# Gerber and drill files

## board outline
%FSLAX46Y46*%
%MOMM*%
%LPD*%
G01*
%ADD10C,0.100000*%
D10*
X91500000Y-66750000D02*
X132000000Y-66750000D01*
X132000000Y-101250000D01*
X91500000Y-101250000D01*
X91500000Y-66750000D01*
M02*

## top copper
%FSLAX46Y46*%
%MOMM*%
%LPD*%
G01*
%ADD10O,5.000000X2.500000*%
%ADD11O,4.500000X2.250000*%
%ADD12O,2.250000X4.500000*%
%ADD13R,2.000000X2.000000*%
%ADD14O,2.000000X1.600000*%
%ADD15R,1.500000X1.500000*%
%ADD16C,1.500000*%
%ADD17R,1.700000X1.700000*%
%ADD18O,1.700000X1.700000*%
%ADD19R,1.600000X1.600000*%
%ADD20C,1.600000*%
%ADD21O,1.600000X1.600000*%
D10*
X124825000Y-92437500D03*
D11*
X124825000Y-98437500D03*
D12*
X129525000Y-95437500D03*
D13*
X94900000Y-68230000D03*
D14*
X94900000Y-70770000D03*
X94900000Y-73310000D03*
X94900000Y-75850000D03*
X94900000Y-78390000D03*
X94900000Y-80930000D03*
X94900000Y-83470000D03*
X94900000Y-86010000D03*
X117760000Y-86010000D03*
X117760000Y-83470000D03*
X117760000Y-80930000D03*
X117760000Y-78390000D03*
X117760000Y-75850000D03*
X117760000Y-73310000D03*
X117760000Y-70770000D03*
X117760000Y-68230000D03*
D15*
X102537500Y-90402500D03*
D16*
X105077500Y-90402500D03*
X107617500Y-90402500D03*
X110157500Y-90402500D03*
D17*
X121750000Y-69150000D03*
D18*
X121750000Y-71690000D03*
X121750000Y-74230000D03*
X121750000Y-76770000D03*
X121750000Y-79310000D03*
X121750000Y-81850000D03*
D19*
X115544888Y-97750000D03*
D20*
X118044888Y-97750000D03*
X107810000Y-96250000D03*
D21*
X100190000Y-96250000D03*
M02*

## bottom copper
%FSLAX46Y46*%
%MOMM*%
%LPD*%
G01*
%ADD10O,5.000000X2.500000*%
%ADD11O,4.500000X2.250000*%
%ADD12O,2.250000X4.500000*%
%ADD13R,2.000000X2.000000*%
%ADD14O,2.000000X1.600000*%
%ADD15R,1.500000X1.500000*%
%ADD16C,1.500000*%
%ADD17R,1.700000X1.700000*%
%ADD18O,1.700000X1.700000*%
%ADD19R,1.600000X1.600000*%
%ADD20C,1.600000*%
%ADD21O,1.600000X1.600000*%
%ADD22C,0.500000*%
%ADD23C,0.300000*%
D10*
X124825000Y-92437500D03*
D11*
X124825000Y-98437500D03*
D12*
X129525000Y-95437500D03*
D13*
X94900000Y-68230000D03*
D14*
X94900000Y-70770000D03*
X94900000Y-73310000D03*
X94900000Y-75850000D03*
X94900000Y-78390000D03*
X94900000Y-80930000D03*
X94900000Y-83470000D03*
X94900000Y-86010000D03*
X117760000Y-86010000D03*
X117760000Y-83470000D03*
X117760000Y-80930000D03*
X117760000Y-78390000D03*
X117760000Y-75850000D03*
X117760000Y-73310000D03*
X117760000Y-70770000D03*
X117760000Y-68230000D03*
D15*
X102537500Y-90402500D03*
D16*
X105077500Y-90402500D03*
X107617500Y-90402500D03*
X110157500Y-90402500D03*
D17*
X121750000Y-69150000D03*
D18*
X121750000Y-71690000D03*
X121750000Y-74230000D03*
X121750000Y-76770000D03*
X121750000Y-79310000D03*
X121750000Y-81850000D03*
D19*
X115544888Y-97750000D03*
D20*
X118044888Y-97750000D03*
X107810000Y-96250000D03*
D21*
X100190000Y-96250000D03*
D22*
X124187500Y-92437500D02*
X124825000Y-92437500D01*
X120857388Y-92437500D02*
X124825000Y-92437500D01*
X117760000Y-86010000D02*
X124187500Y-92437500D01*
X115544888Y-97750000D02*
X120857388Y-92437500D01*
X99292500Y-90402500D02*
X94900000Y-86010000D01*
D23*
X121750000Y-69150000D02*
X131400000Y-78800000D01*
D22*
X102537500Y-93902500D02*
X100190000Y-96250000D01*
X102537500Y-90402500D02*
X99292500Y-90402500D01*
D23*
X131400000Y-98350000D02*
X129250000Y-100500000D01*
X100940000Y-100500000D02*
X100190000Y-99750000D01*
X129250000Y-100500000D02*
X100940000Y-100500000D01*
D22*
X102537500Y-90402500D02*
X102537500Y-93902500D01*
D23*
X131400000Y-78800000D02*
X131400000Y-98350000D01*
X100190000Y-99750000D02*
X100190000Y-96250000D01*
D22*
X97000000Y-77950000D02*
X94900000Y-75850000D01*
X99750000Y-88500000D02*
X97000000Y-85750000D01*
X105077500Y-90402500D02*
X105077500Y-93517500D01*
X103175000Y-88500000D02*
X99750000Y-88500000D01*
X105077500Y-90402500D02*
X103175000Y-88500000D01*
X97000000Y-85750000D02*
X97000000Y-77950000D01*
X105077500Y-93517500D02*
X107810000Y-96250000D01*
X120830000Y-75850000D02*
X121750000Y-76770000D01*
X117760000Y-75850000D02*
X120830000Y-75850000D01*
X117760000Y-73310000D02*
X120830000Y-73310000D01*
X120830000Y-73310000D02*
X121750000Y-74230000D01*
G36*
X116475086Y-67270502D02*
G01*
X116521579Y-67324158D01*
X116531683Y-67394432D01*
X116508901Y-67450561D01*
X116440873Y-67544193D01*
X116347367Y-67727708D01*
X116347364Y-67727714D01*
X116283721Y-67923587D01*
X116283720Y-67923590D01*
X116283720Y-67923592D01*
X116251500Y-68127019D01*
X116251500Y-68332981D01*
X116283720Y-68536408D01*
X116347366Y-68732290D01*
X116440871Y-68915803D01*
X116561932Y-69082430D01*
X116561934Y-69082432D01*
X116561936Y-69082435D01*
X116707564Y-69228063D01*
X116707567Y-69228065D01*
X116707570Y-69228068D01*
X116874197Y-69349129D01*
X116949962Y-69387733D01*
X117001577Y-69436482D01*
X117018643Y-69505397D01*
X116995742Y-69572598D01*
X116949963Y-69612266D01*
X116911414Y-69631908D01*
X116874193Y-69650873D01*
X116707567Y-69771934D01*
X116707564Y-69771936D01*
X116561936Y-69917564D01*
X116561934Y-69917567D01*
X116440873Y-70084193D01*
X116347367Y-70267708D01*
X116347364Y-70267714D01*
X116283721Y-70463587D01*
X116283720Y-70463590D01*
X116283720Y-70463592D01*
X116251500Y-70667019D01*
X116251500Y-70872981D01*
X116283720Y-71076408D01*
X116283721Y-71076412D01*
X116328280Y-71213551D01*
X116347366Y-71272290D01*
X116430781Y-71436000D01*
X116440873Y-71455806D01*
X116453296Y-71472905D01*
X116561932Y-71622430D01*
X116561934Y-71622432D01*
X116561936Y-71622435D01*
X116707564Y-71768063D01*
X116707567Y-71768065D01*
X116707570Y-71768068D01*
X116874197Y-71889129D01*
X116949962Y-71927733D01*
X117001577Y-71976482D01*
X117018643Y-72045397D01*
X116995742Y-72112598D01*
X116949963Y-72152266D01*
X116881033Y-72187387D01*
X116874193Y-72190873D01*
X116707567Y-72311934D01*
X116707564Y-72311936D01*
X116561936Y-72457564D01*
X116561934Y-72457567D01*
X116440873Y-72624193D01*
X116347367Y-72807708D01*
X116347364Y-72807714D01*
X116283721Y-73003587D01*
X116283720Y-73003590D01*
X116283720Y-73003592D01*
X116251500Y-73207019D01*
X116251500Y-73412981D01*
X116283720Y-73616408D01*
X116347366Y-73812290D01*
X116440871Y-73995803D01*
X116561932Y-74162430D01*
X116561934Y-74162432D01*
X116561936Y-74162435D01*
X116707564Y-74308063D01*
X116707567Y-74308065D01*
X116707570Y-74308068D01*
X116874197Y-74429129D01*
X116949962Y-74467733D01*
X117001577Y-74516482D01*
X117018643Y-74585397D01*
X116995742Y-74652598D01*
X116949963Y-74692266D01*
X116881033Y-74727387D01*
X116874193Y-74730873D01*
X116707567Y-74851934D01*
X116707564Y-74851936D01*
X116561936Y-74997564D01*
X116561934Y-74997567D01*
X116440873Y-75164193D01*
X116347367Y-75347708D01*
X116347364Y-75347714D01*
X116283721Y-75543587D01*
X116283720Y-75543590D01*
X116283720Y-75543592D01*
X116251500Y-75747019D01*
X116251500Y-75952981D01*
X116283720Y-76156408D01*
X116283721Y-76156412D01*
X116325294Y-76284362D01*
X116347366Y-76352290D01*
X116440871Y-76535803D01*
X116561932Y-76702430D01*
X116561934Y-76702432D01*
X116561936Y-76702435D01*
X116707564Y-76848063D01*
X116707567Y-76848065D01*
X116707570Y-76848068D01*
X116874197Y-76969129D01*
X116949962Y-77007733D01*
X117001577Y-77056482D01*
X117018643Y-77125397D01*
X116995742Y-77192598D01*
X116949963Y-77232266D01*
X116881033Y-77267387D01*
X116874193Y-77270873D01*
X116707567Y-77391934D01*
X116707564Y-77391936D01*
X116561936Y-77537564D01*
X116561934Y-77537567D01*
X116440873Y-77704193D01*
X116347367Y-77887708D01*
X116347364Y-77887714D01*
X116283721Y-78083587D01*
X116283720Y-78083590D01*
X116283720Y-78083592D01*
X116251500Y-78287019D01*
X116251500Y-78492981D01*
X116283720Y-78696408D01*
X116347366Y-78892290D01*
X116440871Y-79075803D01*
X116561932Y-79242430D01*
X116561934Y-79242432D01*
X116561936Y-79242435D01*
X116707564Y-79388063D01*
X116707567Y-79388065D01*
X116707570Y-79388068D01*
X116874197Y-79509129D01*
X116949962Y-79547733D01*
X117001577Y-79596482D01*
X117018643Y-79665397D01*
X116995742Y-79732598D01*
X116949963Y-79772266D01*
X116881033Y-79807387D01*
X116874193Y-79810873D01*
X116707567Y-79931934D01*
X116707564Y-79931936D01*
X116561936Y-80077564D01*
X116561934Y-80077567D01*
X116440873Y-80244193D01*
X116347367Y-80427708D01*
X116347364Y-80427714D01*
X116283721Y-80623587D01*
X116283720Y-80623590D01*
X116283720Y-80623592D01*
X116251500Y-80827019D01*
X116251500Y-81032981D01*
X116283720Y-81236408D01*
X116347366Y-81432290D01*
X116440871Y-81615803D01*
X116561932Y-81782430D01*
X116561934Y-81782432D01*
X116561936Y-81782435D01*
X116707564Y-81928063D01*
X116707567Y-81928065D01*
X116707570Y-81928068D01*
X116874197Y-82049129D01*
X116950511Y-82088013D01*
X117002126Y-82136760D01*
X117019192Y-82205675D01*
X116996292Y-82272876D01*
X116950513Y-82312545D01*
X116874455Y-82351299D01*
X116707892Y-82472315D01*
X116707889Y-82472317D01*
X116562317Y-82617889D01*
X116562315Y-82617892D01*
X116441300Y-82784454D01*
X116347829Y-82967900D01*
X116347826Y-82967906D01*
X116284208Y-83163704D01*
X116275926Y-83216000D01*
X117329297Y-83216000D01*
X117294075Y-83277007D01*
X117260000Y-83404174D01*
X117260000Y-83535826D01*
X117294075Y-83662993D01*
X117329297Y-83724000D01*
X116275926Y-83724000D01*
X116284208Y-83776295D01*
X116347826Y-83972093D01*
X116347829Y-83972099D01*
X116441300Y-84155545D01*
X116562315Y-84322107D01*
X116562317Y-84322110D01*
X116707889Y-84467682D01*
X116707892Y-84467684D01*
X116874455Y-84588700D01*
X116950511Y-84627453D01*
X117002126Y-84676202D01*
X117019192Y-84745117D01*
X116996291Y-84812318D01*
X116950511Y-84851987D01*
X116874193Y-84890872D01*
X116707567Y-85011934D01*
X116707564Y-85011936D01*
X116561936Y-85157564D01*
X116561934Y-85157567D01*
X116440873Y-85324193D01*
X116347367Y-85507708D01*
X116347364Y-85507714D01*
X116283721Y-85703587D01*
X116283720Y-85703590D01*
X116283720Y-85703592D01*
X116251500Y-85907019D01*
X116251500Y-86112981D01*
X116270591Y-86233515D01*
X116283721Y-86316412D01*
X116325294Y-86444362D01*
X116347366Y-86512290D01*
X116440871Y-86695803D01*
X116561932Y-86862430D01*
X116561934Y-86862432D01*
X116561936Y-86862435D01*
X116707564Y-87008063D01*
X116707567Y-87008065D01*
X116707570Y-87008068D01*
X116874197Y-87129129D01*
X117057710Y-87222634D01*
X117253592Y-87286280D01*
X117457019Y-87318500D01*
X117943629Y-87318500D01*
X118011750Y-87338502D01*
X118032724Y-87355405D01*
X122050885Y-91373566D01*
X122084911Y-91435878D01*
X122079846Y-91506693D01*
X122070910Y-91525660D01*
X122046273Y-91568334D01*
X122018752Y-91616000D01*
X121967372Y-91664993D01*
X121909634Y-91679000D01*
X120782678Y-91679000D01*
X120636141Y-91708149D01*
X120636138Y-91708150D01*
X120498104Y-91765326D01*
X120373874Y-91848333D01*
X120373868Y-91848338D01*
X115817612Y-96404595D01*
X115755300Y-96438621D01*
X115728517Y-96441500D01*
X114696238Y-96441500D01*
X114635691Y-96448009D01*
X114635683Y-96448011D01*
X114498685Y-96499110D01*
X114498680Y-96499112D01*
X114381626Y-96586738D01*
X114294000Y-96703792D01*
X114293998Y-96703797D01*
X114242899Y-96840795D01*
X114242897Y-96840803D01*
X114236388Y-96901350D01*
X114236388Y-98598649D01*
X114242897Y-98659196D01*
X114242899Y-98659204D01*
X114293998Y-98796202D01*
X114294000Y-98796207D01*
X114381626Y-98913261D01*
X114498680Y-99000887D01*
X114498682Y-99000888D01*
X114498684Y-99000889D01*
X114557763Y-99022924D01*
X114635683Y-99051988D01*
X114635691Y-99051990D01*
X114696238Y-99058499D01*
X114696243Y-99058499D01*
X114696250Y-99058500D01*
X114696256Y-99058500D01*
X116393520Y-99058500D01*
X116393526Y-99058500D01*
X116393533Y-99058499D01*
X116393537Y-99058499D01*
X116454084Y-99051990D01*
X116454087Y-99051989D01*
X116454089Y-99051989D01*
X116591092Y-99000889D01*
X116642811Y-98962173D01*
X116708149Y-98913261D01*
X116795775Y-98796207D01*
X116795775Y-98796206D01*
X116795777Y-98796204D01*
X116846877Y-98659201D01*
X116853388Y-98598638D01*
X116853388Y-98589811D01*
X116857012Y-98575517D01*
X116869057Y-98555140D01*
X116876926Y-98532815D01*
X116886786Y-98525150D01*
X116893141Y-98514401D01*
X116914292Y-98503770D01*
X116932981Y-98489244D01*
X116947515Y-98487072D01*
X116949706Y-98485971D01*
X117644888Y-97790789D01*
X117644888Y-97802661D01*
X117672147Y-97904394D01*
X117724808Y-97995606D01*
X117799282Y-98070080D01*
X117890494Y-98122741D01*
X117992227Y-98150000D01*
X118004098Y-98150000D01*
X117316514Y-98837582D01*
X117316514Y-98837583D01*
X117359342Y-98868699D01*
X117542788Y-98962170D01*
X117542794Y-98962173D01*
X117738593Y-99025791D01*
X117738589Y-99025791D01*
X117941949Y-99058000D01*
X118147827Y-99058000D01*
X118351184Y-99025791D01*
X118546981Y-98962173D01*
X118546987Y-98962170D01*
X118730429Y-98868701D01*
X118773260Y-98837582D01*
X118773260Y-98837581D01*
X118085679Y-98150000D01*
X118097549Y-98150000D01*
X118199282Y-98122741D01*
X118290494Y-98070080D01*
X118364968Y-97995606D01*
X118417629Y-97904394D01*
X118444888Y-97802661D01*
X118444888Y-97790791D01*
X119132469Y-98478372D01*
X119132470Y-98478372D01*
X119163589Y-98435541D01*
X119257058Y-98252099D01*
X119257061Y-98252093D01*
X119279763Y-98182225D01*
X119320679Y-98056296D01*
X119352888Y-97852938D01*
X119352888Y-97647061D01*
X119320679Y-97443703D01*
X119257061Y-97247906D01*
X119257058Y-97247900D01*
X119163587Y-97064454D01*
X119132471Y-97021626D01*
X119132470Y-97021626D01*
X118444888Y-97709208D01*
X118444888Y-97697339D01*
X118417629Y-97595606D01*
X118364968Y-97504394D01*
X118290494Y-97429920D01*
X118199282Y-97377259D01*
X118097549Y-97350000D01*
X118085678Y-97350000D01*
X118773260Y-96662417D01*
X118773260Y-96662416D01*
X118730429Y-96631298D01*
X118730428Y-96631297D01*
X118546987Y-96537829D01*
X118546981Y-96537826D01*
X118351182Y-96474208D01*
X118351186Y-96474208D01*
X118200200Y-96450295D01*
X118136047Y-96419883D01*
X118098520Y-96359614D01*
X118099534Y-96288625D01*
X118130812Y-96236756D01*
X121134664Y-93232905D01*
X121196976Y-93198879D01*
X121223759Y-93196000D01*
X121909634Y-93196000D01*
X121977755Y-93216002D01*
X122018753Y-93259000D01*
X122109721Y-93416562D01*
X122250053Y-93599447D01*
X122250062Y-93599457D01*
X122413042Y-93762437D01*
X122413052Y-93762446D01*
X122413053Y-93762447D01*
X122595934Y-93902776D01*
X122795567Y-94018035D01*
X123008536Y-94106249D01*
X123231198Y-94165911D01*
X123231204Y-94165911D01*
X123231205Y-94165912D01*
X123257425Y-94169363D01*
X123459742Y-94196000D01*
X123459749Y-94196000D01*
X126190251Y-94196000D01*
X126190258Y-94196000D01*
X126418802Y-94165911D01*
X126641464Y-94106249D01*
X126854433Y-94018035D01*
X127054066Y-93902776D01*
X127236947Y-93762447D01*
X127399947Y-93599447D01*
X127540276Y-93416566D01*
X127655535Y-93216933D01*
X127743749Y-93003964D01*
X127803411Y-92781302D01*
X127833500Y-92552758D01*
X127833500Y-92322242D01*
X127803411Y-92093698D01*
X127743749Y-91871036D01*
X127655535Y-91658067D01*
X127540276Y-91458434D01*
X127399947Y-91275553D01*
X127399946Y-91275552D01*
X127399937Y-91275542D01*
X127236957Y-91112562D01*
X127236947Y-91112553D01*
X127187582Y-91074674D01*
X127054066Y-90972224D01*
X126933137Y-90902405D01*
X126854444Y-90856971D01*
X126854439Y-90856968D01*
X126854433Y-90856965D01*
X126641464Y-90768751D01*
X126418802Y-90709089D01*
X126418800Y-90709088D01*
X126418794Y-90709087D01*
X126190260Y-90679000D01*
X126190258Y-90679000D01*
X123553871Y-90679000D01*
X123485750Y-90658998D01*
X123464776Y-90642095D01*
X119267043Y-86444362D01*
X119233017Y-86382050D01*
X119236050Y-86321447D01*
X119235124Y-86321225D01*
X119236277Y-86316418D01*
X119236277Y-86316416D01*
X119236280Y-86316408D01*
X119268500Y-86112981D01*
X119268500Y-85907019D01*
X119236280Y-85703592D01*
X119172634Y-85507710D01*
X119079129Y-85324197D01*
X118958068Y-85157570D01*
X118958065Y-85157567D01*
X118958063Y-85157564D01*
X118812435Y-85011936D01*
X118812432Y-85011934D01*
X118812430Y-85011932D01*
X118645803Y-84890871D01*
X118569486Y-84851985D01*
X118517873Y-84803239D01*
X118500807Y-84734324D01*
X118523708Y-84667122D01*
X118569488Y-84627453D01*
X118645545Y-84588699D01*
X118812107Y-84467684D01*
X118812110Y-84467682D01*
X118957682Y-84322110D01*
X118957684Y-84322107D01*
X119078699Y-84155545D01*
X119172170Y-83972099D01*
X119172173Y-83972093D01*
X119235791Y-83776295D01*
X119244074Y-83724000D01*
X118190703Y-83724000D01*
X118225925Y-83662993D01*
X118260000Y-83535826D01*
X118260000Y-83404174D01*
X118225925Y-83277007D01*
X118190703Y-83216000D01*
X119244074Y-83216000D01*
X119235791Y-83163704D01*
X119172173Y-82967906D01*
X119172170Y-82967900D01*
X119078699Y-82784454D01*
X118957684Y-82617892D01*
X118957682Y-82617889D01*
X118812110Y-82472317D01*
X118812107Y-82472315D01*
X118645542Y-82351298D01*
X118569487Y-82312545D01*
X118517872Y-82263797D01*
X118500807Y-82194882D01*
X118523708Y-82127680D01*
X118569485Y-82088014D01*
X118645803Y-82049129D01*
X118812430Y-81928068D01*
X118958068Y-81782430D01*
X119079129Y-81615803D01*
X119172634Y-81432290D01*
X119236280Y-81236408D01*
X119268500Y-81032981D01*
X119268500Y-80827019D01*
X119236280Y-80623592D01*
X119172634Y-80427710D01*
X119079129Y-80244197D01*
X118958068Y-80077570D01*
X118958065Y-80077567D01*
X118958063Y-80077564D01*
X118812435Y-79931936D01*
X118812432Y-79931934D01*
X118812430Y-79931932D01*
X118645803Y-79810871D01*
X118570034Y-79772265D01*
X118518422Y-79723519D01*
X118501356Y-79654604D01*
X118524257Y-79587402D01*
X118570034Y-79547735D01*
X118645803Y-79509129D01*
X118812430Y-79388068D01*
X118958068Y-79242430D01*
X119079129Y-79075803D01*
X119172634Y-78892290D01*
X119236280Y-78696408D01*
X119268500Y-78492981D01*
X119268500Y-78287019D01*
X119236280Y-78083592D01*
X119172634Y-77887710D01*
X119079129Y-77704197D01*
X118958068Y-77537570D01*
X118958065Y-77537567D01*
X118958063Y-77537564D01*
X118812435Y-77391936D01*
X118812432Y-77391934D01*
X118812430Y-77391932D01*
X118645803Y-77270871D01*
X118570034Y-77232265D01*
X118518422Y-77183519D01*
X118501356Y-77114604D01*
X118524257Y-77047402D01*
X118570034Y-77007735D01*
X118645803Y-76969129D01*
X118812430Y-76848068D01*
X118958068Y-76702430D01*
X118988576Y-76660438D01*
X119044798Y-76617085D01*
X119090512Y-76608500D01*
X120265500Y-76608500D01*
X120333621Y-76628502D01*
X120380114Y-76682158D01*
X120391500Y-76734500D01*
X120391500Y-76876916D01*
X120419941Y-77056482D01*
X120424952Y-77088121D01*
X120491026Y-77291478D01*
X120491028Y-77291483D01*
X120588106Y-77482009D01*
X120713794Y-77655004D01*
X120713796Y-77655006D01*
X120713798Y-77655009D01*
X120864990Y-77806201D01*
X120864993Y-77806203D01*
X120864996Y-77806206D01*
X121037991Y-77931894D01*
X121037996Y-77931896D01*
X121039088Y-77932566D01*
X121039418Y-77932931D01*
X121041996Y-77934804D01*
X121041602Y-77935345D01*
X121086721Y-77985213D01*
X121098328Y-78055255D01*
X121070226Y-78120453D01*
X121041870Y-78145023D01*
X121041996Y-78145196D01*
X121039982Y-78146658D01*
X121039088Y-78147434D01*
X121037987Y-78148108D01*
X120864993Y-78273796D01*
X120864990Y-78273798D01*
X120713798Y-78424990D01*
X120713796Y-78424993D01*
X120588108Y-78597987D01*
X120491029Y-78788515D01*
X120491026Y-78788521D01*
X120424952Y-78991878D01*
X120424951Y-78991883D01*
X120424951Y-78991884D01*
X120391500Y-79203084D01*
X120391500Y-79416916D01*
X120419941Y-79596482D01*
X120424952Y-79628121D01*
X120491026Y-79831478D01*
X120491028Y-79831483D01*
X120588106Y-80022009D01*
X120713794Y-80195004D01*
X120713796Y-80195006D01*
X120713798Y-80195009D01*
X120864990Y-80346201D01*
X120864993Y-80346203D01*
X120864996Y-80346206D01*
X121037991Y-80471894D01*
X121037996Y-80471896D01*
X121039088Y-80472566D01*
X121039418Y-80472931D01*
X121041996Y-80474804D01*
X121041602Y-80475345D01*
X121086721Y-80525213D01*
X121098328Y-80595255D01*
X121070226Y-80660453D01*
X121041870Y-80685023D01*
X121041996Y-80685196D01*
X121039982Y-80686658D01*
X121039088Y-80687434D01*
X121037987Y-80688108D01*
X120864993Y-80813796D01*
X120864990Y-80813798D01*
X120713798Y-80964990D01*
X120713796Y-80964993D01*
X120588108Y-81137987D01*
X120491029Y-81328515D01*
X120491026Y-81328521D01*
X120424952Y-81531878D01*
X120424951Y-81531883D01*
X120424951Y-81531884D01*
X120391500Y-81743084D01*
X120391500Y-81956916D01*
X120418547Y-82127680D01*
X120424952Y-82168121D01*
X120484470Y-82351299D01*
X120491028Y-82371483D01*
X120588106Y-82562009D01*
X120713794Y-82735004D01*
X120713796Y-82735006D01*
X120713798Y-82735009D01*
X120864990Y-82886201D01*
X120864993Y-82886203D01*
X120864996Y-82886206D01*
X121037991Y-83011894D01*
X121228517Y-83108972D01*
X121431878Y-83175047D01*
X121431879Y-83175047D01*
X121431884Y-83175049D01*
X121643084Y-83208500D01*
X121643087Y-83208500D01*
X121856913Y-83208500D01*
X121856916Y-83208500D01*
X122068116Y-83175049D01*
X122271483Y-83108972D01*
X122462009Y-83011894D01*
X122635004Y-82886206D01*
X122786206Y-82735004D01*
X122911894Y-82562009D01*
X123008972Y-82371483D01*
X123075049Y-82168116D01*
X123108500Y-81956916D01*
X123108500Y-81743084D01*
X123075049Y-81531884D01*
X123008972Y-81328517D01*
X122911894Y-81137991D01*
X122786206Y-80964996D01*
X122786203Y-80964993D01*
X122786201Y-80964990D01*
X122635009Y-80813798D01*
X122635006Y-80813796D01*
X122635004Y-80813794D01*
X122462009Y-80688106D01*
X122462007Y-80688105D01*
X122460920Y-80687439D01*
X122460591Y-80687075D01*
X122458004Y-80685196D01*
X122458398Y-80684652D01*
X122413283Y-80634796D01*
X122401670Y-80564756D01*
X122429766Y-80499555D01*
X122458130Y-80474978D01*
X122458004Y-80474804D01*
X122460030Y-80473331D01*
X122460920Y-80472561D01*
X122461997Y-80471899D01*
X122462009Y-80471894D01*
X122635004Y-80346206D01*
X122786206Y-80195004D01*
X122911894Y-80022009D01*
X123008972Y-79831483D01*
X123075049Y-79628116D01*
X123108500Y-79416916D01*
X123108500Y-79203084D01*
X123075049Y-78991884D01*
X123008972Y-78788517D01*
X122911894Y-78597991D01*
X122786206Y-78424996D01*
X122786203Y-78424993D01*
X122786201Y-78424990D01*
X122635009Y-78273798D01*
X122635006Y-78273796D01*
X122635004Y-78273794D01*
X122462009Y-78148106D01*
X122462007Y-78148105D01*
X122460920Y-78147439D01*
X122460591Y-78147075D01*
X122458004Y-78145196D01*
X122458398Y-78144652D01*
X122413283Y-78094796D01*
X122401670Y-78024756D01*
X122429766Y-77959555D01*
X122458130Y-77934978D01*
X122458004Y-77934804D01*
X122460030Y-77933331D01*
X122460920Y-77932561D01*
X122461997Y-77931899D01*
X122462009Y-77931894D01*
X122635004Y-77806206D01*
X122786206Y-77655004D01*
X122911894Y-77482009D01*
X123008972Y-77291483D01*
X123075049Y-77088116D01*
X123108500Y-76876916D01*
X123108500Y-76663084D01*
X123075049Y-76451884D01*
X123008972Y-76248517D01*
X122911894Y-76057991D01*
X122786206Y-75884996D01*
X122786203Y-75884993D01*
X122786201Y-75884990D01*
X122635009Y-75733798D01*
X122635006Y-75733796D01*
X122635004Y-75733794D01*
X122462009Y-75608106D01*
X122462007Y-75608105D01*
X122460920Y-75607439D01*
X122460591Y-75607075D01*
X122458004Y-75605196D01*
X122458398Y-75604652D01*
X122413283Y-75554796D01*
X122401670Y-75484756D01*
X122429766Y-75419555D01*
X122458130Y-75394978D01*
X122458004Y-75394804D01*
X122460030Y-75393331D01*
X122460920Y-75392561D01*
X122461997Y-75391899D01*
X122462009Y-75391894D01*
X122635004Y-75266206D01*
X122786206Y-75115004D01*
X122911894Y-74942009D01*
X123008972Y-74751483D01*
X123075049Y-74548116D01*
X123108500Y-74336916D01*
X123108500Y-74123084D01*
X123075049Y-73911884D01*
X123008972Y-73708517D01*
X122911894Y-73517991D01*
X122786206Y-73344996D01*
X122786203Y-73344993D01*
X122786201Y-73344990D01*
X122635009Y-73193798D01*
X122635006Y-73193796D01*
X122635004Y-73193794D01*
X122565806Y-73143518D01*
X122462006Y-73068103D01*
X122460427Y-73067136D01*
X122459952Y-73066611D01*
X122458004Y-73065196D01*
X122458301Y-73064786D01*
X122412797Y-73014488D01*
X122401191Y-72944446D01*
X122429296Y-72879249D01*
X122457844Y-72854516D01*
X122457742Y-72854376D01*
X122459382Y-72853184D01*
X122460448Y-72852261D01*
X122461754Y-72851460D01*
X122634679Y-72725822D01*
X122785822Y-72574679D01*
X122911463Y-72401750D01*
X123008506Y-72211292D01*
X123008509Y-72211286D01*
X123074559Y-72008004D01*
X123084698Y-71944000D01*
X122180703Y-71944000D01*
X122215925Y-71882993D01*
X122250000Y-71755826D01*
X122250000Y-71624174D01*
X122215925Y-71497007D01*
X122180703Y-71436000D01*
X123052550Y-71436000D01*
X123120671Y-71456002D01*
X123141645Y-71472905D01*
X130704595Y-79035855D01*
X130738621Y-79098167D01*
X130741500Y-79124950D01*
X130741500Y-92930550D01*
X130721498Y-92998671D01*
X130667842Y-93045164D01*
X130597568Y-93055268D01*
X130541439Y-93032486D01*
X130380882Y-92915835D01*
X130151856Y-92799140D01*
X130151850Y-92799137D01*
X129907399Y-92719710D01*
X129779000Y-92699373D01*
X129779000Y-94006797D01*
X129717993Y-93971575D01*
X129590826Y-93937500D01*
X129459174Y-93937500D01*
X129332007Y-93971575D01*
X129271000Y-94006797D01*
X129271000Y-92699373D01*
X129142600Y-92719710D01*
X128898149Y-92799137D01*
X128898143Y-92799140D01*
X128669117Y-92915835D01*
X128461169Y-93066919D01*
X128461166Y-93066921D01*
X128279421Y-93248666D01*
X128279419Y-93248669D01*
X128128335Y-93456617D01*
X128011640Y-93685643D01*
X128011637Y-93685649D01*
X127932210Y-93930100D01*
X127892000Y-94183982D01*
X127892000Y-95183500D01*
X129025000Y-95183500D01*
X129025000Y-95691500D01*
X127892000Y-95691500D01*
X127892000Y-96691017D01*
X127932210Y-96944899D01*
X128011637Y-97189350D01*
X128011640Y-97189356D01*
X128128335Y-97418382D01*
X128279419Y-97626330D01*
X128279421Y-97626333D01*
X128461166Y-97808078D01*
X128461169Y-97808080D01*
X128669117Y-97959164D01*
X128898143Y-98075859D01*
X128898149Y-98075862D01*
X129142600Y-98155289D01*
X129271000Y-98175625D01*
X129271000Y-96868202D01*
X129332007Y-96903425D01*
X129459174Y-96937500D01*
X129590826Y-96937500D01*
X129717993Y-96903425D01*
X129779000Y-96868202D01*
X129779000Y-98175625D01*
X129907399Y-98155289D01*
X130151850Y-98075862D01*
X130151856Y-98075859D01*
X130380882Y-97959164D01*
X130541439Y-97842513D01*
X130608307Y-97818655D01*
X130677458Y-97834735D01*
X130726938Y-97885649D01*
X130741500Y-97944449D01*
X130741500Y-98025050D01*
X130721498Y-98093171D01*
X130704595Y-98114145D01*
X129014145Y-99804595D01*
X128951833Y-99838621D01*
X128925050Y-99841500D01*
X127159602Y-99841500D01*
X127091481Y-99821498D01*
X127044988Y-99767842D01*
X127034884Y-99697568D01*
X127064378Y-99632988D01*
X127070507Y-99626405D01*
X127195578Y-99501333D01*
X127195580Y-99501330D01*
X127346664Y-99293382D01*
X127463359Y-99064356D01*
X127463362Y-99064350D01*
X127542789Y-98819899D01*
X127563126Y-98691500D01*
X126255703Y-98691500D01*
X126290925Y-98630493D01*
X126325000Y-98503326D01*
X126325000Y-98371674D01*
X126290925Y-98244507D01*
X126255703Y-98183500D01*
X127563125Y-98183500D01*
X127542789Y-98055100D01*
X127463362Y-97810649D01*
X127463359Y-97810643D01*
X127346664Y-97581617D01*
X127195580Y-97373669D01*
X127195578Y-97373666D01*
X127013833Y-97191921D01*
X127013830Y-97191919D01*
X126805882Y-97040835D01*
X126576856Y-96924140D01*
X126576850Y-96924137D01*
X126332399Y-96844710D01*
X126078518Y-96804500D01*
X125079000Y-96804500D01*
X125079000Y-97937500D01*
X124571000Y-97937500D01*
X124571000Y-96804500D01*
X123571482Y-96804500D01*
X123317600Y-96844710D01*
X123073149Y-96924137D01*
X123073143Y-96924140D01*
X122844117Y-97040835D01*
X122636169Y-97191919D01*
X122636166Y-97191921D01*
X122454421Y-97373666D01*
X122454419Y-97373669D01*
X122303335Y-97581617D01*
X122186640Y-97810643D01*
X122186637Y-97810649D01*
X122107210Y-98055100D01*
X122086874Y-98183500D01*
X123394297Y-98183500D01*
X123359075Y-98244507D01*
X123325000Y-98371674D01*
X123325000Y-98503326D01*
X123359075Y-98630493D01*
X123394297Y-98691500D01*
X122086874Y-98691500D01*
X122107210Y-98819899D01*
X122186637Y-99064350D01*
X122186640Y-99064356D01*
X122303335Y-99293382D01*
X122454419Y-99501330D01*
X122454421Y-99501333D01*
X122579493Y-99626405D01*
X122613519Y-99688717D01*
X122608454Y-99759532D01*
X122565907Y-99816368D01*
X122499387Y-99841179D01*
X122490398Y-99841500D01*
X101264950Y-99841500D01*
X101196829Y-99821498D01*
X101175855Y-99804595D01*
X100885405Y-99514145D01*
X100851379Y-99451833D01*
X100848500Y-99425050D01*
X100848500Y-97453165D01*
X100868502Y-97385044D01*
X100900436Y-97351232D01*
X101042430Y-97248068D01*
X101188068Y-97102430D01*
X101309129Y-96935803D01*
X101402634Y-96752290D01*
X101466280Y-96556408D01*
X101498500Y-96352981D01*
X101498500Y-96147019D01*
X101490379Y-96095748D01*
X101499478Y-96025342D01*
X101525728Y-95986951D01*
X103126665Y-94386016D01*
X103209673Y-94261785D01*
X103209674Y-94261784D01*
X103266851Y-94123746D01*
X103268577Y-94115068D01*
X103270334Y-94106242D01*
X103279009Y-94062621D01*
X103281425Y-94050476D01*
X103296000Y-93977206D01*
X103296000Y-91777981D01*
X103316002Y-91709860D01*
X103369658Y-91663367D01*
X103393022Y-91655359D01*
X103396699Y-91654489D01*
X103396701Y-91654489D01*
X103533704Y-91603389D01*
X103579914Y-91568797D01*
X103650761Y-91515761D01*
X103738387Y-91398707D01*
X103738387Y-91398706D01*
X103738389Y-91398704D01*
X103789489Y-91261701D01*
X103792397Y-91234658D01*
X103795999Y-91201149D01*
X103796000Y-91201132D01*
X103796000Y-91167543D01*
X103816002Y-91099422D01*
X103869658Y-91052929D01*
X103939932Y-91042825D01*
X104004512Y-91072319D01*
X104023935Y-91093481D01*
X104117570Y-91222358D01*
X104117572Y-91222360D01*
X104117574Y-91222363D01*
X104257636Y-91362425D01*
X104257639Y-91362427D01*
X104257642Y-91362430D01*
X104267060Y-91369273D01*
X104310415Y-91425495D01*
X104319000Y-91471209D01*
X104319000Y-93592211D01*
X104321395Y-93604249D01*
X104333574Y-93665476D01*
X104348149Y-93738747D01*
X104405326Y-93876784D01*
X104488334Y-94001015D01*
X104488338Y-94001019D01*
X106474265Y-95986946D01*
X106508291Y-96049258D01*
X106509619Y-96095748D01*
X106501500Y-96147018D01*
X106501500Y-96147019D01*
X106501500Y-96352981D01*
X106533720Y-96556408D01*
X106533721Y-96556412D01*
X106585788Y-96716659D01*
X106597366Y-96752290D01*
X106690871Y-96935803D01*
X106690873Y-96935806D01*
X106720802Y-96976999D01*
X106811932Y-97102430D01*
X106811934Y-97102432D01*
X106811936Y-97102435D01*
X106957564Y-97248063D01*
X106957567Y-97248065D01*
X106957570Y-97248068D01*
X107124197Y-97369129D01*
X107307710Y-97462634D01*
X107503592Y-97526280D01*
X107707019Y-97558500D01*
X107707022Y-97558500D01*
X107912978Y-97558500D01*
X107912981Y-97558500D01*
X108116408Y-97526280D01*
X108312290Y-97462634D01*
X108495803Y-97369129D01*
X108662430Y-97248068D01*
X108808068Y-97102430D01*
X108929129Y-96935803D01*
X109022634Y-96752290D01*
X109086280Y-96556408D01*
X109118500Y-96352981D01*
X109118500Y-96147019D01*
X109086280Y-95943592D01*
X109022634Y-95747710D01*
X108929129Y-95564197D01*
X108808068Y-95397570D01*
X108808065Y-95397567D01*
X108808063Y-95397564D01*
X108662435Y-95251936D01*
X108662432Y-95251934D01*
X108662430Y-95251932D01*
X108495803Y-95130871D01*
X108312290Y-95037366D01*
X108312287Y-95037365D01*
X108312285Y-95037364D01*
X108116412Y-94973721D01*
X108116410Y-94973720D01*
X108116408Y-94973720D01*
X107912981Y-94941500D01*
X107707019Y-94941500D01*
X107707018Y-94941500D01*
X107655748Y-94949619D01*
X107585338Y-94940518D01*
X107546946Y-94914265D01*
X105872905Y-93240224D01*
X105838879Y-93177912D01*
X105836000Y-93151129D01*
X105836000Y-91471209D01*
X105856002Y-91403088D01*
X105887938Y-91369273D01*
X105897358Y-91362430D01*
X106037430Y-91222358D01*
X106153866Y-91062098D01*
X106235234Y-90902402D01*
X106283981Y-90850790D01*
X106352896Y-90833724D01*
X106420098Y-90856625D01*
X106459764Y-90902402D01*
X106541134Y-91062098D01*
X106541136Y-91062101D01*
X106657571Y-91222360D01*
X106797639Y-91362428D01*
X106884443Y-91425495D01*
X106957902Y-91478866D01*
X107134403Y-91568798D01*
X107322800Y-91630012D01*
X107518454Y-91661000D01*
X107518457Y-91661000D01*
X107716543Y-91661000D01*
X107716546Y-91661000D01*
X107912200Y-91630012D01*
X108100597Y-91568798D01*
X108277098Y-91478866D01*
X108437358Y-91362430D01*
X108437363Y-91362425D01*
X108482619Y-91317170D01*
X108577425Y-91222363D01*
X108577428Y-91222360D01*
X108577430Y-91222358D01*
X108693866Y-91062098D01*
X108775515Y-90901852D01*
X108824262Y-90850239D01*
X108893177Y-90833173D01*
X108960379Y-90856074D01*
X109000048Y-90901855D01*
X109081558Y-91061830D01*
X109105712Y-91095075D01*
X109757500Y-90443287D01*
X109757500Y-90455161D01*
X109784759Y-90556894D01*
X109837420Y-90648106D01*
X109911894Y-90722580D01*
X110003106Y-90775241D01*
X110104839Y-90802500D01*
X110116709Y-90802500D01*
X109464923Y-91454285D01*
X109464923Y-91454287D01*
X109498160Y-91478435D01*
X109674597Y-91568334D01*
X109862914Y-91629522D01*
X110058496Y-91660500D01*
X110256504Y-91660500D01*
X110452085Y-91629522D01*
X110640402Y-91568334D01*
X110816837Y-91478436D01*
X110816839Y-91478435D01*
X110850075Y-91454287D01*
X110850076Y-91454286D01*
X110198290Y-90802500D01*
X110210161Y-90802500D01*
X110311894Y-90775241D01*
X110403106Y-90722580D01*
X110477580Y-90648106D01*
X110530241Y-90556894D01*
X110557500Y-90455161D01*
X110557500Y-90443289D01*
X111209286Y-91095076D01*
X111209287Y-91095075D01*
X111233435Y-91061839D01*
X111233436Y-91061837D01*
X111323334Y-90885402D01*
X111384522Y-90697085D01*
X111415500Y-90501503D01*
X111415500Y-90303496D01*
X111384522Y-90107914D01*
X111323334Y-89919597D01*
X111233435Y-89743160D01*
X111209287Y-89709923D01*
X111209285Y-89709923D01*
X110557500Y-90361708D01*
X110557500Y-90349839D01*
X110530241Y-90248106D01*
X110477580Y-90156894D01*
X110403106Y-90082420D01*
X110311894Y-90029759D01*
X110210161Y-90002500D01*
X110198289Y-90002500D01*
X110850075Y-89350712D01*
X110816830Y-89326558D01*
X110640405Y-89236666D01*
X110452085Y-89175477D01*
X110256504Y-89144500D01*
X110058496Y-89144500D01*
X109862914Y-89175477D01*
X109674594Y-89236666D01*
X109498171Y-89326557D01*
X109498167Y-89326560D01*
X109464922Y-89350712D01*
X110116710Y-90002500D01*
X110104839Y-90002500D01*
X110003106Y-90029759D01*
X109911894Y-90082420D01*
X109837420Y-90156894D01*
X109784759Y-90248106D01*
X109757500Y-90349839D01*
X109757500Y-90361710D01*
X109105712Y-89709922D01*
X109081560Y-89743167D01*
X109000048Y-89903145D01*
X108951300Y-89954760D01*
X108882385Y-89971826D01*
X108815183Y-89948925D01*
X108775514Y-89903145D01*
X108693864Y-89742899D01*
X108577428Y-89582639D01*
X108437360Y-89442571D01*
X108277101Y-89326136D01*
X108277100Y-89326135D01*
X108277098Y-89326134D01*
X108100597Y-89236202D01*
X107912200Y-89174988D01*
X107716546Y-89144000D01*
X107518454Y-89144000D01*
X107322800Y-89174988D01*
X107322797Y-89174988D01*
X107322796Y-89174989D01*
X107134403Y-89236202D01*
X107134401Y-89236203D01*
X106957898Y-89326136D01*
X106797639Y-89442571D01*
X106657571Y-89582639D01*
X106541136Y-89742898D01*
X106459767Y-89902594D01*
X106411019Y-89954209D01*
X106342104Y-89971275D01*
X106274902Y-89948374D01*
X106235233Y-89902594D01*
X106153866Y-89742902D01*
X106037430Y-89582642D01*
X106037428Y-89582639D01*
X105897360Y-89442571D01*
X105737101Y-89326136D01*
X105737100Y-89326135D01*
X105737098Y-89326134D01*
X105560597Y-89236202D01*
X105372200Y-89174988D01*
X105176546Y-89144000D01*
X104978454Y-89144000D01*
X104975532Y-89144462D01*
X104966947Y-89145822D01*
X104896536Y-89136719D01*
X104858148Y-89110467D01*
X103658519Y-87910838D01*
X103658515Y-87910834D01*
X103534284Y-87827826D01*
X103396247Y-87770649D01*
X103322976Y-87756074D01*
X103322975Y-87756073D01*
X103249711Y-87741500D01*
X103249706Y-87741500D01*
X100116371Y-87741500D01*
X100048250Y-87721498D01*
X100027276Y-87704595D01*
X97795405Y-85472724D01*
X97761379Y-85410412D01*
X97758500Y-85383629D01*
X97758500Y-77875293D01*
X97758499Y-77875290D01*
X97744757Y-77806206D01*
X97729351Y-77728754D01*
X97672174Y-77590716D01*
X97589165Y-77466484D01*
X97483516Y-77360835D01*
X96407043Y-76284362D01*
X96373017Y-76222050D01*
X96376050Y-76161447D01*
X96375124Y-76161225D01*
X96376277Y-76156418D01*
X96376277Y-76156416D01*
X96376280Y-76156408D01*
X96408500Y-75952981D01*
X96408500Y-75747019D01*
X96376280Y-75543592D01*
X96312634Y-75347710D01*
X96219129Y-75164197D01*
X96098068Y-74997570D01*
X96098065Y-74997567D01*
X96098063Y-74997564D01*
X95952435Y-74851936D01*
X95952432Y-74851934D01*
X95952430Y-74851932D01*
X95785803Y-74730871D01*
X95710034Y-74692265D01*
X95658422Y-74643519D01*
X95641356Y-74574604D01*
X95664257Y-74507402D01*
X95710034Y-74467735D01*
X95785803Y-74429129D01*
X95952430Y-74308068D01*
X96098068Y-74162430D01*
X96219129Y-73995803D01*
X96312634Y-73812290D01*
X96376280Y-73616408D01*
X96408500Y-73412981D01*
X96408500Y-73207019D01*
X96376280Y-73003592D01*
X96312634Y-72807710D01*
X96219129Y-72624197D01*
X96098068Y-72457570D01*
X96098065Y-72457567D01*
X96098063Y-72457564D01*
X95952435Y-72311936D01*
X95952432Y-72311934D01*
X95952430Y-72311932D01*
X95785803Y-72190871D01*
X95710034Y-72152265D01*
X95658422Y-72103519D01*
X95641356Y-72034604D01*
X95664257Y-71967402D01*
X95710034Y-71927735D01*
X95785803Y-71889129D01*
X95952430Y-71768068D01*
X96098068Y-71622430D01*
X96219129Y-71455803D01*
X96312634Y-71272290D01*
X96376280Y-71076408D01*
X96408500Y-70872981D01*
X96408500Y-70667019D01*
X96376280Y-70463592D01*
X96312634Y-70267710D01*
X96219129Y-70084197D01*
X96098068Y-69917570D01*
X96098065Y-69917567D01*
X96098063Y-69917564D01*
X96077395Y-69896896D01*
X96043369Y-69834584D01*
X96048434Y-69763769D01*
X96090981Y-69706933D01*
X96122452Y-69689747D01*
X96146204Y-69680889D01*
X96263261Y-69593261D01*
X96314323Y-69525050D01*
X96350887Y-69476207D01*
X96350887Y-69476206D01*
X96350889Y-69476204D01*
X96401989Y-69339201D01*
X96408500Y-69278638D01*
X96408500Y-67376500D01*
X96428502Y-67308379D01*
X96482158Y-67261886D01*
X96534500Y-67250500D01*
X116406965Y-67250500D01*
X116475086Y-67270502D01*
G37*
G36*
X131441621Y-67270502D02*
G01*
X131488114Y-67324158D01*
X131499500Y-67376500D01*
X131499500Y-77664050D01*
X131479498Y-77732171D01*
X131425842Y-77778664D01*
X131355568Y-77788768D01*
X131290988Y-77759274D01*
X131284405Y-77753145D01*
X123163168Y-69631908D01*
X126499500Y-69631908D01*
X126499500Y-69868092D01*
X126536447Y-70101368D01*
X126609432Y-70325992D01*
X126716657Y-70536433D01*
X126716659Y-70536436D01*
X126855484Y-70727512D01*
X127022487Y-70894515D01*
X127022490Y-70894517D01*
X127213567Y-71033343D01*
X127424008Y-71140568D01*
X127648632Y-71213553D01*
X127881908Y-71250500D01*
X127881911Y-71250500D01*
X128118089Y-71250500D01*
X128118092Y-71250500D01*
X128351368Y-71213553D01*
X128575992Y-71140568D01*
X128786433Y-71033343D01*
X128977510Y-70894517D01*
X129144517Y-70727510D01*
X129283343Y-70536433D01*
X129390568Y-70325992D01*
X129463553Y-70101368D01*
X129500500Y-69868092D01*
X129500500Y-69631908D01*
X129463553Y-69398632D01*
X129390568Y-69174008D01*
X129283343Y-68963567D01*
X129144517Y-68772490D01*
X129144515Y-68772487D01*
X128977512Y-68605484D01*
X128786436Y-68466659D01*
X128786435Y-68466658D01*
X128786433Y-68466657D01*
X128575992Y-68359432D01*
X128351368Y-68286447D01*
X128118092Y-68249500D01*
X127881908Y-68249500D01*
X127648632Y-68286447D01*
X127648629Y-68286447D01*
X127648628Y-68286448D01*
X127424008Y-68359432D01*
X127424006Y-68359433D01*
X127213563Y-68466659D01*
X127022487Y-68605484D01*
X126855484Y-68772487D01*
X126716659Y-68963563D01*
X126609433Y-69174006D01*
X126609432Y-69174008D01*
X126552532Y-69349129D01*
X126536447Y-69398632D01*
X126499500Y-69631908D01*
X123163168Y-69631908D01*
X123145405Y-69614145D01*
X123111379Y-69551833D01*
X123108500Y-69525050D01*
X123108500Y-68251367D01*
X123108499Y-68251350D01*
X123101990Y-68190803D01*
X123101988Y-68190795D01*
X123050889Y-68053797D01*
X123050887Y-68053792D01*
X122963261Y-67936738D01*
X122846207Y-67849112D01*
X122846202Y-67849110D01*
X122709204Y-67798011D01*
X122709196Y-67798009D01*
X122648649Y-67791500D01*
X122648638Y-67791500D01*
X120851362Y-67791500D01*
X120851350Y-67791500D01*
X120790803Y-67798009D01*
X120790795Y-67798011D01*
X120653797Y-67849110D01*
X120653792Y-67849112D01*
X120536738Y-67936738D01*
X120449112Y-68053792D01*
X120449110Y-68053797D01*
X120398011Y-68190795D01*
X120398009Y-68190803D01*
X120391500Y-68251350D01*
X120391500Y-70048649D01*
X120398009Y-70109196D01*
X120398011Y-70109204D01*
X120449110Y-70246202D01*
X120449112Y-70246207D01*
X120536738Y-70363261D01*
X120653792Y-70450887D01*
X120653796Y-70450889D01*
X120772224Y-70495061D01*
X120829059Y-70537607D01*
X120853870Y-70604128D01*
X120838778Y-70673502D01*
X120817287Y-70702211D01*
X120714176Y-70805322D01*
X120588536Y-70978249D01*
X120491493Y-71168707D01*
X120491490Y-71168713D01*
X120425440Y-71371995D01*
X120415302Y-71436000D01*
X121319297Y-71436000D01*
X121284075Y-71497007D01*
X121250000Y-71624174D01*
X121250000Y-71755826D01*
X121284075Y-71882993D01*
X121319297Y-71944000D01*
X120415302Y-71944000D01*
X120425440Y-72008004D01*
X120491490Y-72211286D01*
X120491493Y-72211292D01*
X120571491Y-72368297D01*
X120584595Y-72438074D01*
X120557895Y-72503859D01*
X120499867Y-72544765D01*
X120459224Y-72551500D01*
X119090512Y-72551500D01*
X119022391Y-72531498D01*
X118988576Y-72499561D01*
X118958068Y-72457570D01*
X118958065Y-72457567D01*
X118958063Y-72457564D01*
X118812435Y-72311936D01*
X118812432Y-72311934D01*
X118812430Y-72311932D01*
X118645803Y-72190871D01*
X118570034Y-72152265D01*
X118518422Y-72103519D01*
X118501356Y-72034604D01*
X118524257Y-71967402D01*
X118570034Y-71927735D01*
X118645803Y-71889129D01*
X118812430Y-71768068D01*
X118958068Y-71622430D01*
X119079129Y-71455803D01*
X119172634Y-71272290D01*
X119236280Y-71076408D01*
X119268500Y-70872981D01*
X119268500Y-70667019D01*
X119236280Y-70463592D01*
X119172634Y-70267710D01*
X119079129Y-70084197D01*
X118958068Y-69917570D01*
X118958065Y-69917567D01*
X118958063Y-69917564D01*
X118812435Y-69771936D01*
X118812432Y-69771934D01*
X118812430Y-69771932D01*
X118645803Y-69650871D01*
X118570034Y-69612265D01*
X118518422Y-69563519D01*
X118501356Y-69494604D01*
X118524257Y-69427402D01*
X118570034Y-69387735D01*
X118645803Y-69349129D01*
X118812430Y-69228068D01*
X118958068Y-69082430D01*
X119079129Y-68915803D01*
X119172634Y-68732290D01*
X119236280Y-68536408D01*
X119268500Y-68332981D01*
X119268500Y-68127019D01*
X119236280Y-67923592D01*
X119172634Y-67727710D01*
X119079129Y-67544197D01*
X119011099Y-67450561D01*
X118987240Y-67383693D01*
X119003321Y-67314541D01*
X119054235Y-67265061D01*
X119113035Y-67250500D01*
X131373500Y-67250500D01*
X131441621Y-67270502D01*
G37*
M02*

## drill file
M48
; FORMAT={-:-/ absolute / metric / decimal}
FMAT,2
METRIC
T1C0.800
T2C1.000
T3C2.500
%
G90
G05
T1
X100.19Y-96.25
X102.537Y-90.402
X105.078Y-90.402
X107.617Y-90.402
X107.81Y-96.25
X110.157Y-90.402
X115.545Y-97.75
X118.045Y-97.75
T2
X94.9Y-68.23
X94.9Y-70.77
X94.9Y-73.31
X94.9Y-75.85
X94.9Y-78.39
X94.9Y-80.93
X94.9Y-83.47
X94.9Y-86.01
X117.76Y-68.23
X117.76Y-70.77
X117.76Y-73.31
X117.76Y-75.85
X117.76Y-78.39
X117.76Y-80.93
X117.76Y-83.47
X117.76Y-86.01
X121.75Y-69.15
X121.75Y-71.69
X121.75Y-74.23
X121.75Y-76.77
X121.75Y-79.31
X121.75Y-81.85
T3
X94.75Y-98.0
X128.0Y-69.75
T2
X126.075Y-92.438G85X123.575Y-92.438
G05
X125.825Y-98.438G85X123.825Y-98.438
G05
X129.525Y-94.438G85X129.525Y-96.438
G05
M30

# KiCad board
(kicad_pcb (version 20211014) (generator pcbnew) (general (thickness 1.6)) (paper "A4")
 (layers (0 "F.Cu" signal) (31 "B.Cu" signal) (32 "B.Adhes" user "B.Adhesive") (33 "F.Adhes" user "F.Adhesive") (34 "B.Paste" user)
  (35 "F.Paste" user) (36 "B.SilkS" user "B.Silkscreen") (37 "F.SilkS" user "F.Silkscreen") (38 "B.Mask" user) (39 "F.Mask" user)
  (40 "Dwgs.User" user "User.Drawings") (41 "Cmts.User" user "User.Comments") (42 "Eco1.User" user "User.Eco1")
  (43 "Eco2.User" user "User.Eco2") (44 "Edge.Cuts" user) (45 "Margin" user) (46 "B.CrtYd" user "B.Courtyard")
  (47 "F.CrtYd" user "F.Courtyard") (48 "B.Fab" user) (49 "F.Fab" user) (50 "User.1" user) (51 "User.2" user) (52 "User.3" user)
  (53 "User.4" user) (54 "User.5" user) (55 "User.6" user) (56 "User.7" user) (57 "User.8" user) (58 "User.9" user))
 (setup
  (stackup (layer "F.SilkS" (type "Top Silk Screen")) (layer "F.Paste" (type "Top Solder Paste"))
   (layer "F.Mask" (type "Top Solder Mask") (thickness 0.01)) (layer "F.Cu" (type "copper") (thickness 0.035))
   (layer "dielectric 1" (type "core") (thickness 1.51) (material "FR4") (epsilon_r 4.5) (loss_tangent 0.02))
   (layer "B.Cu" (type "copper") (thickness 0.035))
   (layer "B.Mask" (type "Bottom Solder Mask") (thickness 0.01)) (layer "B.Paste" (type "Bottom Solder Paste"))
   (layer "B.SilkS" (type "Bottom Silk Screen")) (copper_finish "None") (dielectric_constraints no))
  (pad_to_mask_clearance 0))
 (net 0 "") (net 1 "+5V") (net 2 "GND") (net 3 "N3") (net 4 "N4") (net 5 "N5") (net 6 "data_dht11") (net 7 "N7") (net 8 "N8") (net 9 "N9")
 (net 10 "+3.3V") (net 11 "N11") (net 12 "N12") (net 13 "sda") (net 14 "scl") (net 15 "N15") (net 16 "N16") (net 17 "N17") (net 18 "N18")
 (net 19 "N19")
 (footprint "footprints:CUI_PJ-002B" (layer "F.Cu") (at 124.825 92.4375 -90)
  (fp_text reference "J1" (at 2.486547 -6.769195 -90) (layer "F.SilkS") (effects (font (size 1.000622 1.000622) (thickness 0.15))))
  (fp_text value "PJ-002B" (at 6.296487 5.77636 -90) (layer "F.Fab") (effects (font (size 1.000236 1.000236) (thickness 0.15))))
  (pad "1" thru_hole oval locked (at 0 0 270) (size 2.5 5) (drill oval 1 3.5) (layers *.Cu *.Mask) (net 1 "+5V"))
  (pad "2" thru_hole oval locked (at 6 0 270) (size 2.25 4.5) (drill oval 1 3) (layers *.Cu *.Mask) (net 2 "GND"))
  (pad "3" thru_hole oval locked (at 3 -4.7 270) (size 4.5 2.25) (drill oval 3 1) (layers *.Cu *.Mask) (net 2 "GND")))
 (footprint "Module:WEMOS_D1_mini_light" (layer "F.Cu") (at 94.9 68.23)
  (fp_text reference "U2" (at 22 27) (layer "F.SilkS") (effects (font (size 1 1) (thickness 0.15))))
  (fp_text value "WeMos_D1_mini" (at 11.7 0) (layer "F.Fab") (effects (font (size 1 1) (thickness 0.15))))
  (pad "1" thru_hole rect (at 0 0) (size 2 2) (drill 1) (layers *.Cu *.Mask) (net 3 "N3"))
  (pad "2" thru_hole oval (at 0 2.54) (size 2 1.6) (drill 1) (layers *.Cu *.Mask) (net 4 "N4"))
  (pad "3" thru_hole oval (at 0 5.08) (size 2 1.6) (drill 1) (layers *.Cu *.Mask) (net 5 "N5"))
  (pad "4" thru_hole oval (at 0 7.62) (size 2 1.6) (drill 1) (layers *.Cu *.Mask) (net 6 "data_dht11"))
  (pad "5" thru_hole oval (at 0 10.16) (size 2 1.6) (drill 1) (layers *.Cu *.Mask) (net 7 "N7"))
  (pad "6" thru_hole oval (at 0 12.7) (size 2 1.6) (drill 1) (layers *.Cu *.Mask) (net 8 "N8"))
  (pad "7" thru_hole oval (at 0 15.24) (size 2 1.6) (drill 1) (layers *.Cu *.Mask) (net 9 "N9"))
  (pad "8" thru_hole oval (at 0 17.78) (size 2 1.6) (drill 1) (layers *.Cu *.Mask) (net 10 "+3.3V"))
  (pad "9" thru_hole oval (at 22.86 17.78) (size 2 1.6) (drill 1) (layers *.Cu *.Mask) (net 1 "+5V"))
  (pad "10" thru_hole oval (at 22.86 15.24) (size 2 1.6) (drill 1) (layers *.Cu *.Mask) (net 2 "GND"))
  (pad "11" thru_hole oval (at 22.86 12.7) (size 2 1.6) (drill 1) (layers *.Cu *.Mask) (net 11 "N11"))
  (pad "12" thru_hole oval (at 22.86 10.16) (size 2 1.6) (drill 1) (layers *.Cu *.Mask) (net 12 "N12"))
  (pad "13" thru_hole oval (at 22.86 7.62) (size 2 1.6) (drill 1) (layers *.Cu *.Mask) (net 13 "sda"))
  (pad "14" thru_hole oval (at 22.86 5.08) (size 2 1.6) (drill 1) (layers *.Cu *.Mask) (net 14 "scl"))
  (pad "15" thru_hole oval (at 22.86 2.54) (size 2 1.6) (drill 1) (layers *.Cu *.Mask) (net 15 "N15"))
  (pad "16" thru_hole oval (at 22.86 0) (size 2 1.6) (drill 1) (layers *.Cu *.Mask) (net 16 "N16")))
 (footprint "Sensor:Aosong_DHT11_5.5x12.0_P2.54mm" (layer "F.Cu") (at 102.5375 90.4025 90)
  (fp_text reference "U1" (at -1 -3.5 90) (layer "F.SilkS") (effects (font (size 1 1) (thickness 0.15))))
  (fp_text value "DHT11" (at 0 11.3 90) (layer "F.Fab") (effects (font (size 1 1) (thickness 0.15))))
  (pad "1" thru_hole rect (at 0 0 90) (size 1.5 1.5) (drill 0.8) (layers *.Cu *.Mask) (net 10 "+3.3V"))
  (pad "2" thru_hole circle (at 0 2.54 90) (size 1.5 1.5) (drill 0.8) (layers *.Cu *.Mask) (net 6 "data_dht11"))
  (pad "3" thru_hole circle (at 0 5.08 90) (size 1.5 1.5) (drill 0.8) (layers *.Cu *.Mask) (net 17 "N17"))
  (pad "4" thru_hole circle (at 0 7.62 90) (size 1.5 1.5) (drill 0.8) (layers *.Cu *.Mask) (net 2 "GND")))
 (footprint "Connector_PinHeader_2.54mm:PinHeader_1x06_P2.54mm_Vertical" (layer "F.Cu") (at 121.75 69.15)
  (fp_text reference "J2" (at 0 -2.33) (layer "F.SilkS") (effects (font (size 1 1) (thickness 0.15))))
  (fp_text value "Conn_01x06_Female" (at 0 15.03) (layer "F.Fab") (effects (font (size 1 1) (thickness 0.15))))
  (pad "1" thru_hole rect (at 0 0) (size 1.7 1.7) (drill 1) (layers *.Cu *.Mask) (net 10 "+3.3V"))
  (pad "2" thru_hole oval (at 0 2.54) (size 1.7 1.7) (drill 1) (layers *.Cu *.Mask) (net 2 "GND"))
  (pad "3" thru_hole oval (at 0 5.08) (size 1.7 1.7) (drill 1) (layers *.Cu *.Mask) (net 14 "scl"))
  (pad "4" thru_hole oval (at 0 7.62) (size 1.7 1.7) (drill 1) (layers *.Cu *.Mask) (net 13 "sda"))
  (pad "5" thru_hole oval (at 0 10.16) (size 1.7 1.7) (drill 1) (layers *.Cu *.Mask) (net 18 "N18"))
  (pad "6" thru_hole oval (at 0 12.7) (size 1.7 1.7) (drill 1) (layers *.Cu *.Mask) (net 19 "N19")))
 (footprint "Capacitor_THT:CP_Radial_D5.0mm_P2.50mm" (layer "F.Cu") (at 115.544888 97.75)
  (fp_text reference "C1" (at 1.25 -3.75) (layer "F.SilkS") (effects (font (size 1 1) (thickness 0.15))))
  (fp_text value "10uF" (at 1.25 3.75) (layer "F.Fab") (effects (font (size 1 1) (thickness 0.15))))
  (pad "1" thru_hole rect (at 0 0) (size 1.6 1.6) (drill 0.8) (layers *.Cu *.Mask) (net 1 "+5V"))
  (pad "2" thru_hole circle (at 2.5 0) (size 1.6 1.6) (drill 0.8) (layers *.Cu *.Mask) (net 2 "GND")))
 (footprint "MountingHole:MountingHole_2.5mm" (layer "F.Cu") (at 94.75 98)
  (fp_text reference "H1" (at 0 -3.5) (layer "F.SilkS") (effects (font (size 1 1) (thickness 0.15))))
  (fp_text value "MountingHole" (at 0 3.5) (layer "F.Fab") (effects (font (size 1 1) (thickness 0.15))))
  (pad "" np_thru_hole circle (at 0 0) (size 2.5 2.5) (drill 2.5) (layers *.Cu *.Mask)))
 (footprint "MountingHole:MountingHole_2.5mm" (layer "F.Cu") (at 128 69.75)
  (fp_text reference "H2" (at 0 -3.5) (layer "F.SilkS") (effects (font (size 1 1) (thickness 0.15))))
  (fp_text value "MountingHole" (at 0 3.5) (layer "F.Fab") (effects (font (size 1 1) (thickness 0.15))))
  (pad "" np_thru_hole circle (at 0 0) (size 2.5 2.5) (drill 2.5) (layers *.Cu *.Mask)))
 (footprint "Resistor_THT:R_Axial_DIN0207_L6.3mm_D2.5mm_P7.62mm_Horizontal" (layer "F.Cu") (at 107.81 96.25 180)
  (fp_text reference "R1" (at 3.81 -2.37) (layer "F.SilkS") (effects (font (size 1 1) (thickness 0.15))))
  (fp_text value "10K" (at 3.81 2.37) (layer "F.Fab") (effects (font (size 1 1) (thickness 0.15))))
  (pad "1" thru_hole circle (at 0 0 180) (size 1.6 1.6) (drill 0.8) (layers *.Cu *.Mask) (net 6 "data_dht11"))
  (pad "2" thru_hole oval (at 7.62 0 180) (size 1.6 1.6) (drill 0.8) (layers *.Cu *.Mask) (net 10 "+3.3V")))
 (gr_rect (start 91.5 66.75) (end 132 101.25) (layer "Edge.Cuts") (width 0.1) (fill none))
 (segment (start 124.1875 92.4375) (end 124.825 92.4375) (width 0.5) (layer "B.Cu") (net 1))
 (segment (start 120.857388 92.4375) (end 124.825 92.4375) (width 0.5) (layer "B.Cu") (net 1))
 (segment (start 117.76 86.01) (end 124.1875 92.4375) (width 0.5) (layer "B.Cu") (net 1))
 (segment (start 115.544888 97.75) (end 120.857388 92.4375) (width 0.5) (layer "B.Cu") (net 1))
 (segment (start 99.2925 90.4025) (end 94.9 86.01) (width 0.5) (layer "B.Cu") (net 10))
 (segment (start 121.75 69.15) (end 131.4 78.8) (width 0.3) (layer "B.Cu") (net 10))
 (segment (start 102.5375 93.9025) (end 100.19 96.25) (width 0.5) (layer "B.Cu") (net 10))
 (segment (start 102.5375 90.4025) (end 99.2925 90.4025) (width 0.5) (layer "B.Cu") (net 10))
 (segment (start 131.4 98.35) (end 129.25 100.5) (width 0.3) (layer "B.Cu") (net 10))
 (segment (start 100.94 100.5) (end 100.19 99.75) (width 0.3) (layer "B.Cu") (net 10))
 (segment (start 129.25 100.5) (end 100.94 100.5) (width 0.3) (layer "B.Cu") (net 10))
 (segment (start 102.5375 90.4025) (end 102.5375 93.9025) (width 0.5) (layer "B.Cu") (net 10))
 (segment (start 131.4 78.8) (end 131.4 98.35) (width 0.3) (layer "B.Cu") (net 10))
 (segment (start 100.19 99.75) (end 100.19 96.25) (width 0.3) (layer "B.Cu") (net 10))
 (segment (start 97 77.95) (end 94.9 75.85) (width 0.5) (layer "B.Cu") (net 6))
 (segment (start 99.75 88.5) (end 97 85.75) (width 0.5) (layer "B.Cu") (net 6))
 (segment (start 105.0775 90.4025) (end 105.0775 93.5175) (width 0.5) (layer "B.Cu") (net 6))
 (segment (start 103.175 88.5) (end 99.75 88.5) (width 0.5) (layer "B.Cu") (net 6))
 (segment (start 105.0775 90.4025) (end 103.175 88.5) (width 0.5) (layer "B.Cu") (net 6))
 (segment (start 97 85.75) (end 97 77.95) (width 0.5) (layer "B.Cu") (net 6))
 (segment (start 105.0775 93.5175) (end 107.81 96.25) (width 0.5) (layer "B.Cu") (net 6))
 (segment (start 120.83 75.85) (end 121.75 76.77) (width 0.5) (layer "B.Cu") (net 13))
 (segment (start 117.76 75.85) (end 120.83 75.85) (width 0.5) (layer "B.Cu") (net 13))
 (segment (start 117.76 73.31) (end 120.83 73.31) (width 0.5) (layer "B.Cu") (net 14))
 (segment (start 120.83 73.31) (end 121.75 74.23) (width 0.5) (layer "B.Cu") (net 14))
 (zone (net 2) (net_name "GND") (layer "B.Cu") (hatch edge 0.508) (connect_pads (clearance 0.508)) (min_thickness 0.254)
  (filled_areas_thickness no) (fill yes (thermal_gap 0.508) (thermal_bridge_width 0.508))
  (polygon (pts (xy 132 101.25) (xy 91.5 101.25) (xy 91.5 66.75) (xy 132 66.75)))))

